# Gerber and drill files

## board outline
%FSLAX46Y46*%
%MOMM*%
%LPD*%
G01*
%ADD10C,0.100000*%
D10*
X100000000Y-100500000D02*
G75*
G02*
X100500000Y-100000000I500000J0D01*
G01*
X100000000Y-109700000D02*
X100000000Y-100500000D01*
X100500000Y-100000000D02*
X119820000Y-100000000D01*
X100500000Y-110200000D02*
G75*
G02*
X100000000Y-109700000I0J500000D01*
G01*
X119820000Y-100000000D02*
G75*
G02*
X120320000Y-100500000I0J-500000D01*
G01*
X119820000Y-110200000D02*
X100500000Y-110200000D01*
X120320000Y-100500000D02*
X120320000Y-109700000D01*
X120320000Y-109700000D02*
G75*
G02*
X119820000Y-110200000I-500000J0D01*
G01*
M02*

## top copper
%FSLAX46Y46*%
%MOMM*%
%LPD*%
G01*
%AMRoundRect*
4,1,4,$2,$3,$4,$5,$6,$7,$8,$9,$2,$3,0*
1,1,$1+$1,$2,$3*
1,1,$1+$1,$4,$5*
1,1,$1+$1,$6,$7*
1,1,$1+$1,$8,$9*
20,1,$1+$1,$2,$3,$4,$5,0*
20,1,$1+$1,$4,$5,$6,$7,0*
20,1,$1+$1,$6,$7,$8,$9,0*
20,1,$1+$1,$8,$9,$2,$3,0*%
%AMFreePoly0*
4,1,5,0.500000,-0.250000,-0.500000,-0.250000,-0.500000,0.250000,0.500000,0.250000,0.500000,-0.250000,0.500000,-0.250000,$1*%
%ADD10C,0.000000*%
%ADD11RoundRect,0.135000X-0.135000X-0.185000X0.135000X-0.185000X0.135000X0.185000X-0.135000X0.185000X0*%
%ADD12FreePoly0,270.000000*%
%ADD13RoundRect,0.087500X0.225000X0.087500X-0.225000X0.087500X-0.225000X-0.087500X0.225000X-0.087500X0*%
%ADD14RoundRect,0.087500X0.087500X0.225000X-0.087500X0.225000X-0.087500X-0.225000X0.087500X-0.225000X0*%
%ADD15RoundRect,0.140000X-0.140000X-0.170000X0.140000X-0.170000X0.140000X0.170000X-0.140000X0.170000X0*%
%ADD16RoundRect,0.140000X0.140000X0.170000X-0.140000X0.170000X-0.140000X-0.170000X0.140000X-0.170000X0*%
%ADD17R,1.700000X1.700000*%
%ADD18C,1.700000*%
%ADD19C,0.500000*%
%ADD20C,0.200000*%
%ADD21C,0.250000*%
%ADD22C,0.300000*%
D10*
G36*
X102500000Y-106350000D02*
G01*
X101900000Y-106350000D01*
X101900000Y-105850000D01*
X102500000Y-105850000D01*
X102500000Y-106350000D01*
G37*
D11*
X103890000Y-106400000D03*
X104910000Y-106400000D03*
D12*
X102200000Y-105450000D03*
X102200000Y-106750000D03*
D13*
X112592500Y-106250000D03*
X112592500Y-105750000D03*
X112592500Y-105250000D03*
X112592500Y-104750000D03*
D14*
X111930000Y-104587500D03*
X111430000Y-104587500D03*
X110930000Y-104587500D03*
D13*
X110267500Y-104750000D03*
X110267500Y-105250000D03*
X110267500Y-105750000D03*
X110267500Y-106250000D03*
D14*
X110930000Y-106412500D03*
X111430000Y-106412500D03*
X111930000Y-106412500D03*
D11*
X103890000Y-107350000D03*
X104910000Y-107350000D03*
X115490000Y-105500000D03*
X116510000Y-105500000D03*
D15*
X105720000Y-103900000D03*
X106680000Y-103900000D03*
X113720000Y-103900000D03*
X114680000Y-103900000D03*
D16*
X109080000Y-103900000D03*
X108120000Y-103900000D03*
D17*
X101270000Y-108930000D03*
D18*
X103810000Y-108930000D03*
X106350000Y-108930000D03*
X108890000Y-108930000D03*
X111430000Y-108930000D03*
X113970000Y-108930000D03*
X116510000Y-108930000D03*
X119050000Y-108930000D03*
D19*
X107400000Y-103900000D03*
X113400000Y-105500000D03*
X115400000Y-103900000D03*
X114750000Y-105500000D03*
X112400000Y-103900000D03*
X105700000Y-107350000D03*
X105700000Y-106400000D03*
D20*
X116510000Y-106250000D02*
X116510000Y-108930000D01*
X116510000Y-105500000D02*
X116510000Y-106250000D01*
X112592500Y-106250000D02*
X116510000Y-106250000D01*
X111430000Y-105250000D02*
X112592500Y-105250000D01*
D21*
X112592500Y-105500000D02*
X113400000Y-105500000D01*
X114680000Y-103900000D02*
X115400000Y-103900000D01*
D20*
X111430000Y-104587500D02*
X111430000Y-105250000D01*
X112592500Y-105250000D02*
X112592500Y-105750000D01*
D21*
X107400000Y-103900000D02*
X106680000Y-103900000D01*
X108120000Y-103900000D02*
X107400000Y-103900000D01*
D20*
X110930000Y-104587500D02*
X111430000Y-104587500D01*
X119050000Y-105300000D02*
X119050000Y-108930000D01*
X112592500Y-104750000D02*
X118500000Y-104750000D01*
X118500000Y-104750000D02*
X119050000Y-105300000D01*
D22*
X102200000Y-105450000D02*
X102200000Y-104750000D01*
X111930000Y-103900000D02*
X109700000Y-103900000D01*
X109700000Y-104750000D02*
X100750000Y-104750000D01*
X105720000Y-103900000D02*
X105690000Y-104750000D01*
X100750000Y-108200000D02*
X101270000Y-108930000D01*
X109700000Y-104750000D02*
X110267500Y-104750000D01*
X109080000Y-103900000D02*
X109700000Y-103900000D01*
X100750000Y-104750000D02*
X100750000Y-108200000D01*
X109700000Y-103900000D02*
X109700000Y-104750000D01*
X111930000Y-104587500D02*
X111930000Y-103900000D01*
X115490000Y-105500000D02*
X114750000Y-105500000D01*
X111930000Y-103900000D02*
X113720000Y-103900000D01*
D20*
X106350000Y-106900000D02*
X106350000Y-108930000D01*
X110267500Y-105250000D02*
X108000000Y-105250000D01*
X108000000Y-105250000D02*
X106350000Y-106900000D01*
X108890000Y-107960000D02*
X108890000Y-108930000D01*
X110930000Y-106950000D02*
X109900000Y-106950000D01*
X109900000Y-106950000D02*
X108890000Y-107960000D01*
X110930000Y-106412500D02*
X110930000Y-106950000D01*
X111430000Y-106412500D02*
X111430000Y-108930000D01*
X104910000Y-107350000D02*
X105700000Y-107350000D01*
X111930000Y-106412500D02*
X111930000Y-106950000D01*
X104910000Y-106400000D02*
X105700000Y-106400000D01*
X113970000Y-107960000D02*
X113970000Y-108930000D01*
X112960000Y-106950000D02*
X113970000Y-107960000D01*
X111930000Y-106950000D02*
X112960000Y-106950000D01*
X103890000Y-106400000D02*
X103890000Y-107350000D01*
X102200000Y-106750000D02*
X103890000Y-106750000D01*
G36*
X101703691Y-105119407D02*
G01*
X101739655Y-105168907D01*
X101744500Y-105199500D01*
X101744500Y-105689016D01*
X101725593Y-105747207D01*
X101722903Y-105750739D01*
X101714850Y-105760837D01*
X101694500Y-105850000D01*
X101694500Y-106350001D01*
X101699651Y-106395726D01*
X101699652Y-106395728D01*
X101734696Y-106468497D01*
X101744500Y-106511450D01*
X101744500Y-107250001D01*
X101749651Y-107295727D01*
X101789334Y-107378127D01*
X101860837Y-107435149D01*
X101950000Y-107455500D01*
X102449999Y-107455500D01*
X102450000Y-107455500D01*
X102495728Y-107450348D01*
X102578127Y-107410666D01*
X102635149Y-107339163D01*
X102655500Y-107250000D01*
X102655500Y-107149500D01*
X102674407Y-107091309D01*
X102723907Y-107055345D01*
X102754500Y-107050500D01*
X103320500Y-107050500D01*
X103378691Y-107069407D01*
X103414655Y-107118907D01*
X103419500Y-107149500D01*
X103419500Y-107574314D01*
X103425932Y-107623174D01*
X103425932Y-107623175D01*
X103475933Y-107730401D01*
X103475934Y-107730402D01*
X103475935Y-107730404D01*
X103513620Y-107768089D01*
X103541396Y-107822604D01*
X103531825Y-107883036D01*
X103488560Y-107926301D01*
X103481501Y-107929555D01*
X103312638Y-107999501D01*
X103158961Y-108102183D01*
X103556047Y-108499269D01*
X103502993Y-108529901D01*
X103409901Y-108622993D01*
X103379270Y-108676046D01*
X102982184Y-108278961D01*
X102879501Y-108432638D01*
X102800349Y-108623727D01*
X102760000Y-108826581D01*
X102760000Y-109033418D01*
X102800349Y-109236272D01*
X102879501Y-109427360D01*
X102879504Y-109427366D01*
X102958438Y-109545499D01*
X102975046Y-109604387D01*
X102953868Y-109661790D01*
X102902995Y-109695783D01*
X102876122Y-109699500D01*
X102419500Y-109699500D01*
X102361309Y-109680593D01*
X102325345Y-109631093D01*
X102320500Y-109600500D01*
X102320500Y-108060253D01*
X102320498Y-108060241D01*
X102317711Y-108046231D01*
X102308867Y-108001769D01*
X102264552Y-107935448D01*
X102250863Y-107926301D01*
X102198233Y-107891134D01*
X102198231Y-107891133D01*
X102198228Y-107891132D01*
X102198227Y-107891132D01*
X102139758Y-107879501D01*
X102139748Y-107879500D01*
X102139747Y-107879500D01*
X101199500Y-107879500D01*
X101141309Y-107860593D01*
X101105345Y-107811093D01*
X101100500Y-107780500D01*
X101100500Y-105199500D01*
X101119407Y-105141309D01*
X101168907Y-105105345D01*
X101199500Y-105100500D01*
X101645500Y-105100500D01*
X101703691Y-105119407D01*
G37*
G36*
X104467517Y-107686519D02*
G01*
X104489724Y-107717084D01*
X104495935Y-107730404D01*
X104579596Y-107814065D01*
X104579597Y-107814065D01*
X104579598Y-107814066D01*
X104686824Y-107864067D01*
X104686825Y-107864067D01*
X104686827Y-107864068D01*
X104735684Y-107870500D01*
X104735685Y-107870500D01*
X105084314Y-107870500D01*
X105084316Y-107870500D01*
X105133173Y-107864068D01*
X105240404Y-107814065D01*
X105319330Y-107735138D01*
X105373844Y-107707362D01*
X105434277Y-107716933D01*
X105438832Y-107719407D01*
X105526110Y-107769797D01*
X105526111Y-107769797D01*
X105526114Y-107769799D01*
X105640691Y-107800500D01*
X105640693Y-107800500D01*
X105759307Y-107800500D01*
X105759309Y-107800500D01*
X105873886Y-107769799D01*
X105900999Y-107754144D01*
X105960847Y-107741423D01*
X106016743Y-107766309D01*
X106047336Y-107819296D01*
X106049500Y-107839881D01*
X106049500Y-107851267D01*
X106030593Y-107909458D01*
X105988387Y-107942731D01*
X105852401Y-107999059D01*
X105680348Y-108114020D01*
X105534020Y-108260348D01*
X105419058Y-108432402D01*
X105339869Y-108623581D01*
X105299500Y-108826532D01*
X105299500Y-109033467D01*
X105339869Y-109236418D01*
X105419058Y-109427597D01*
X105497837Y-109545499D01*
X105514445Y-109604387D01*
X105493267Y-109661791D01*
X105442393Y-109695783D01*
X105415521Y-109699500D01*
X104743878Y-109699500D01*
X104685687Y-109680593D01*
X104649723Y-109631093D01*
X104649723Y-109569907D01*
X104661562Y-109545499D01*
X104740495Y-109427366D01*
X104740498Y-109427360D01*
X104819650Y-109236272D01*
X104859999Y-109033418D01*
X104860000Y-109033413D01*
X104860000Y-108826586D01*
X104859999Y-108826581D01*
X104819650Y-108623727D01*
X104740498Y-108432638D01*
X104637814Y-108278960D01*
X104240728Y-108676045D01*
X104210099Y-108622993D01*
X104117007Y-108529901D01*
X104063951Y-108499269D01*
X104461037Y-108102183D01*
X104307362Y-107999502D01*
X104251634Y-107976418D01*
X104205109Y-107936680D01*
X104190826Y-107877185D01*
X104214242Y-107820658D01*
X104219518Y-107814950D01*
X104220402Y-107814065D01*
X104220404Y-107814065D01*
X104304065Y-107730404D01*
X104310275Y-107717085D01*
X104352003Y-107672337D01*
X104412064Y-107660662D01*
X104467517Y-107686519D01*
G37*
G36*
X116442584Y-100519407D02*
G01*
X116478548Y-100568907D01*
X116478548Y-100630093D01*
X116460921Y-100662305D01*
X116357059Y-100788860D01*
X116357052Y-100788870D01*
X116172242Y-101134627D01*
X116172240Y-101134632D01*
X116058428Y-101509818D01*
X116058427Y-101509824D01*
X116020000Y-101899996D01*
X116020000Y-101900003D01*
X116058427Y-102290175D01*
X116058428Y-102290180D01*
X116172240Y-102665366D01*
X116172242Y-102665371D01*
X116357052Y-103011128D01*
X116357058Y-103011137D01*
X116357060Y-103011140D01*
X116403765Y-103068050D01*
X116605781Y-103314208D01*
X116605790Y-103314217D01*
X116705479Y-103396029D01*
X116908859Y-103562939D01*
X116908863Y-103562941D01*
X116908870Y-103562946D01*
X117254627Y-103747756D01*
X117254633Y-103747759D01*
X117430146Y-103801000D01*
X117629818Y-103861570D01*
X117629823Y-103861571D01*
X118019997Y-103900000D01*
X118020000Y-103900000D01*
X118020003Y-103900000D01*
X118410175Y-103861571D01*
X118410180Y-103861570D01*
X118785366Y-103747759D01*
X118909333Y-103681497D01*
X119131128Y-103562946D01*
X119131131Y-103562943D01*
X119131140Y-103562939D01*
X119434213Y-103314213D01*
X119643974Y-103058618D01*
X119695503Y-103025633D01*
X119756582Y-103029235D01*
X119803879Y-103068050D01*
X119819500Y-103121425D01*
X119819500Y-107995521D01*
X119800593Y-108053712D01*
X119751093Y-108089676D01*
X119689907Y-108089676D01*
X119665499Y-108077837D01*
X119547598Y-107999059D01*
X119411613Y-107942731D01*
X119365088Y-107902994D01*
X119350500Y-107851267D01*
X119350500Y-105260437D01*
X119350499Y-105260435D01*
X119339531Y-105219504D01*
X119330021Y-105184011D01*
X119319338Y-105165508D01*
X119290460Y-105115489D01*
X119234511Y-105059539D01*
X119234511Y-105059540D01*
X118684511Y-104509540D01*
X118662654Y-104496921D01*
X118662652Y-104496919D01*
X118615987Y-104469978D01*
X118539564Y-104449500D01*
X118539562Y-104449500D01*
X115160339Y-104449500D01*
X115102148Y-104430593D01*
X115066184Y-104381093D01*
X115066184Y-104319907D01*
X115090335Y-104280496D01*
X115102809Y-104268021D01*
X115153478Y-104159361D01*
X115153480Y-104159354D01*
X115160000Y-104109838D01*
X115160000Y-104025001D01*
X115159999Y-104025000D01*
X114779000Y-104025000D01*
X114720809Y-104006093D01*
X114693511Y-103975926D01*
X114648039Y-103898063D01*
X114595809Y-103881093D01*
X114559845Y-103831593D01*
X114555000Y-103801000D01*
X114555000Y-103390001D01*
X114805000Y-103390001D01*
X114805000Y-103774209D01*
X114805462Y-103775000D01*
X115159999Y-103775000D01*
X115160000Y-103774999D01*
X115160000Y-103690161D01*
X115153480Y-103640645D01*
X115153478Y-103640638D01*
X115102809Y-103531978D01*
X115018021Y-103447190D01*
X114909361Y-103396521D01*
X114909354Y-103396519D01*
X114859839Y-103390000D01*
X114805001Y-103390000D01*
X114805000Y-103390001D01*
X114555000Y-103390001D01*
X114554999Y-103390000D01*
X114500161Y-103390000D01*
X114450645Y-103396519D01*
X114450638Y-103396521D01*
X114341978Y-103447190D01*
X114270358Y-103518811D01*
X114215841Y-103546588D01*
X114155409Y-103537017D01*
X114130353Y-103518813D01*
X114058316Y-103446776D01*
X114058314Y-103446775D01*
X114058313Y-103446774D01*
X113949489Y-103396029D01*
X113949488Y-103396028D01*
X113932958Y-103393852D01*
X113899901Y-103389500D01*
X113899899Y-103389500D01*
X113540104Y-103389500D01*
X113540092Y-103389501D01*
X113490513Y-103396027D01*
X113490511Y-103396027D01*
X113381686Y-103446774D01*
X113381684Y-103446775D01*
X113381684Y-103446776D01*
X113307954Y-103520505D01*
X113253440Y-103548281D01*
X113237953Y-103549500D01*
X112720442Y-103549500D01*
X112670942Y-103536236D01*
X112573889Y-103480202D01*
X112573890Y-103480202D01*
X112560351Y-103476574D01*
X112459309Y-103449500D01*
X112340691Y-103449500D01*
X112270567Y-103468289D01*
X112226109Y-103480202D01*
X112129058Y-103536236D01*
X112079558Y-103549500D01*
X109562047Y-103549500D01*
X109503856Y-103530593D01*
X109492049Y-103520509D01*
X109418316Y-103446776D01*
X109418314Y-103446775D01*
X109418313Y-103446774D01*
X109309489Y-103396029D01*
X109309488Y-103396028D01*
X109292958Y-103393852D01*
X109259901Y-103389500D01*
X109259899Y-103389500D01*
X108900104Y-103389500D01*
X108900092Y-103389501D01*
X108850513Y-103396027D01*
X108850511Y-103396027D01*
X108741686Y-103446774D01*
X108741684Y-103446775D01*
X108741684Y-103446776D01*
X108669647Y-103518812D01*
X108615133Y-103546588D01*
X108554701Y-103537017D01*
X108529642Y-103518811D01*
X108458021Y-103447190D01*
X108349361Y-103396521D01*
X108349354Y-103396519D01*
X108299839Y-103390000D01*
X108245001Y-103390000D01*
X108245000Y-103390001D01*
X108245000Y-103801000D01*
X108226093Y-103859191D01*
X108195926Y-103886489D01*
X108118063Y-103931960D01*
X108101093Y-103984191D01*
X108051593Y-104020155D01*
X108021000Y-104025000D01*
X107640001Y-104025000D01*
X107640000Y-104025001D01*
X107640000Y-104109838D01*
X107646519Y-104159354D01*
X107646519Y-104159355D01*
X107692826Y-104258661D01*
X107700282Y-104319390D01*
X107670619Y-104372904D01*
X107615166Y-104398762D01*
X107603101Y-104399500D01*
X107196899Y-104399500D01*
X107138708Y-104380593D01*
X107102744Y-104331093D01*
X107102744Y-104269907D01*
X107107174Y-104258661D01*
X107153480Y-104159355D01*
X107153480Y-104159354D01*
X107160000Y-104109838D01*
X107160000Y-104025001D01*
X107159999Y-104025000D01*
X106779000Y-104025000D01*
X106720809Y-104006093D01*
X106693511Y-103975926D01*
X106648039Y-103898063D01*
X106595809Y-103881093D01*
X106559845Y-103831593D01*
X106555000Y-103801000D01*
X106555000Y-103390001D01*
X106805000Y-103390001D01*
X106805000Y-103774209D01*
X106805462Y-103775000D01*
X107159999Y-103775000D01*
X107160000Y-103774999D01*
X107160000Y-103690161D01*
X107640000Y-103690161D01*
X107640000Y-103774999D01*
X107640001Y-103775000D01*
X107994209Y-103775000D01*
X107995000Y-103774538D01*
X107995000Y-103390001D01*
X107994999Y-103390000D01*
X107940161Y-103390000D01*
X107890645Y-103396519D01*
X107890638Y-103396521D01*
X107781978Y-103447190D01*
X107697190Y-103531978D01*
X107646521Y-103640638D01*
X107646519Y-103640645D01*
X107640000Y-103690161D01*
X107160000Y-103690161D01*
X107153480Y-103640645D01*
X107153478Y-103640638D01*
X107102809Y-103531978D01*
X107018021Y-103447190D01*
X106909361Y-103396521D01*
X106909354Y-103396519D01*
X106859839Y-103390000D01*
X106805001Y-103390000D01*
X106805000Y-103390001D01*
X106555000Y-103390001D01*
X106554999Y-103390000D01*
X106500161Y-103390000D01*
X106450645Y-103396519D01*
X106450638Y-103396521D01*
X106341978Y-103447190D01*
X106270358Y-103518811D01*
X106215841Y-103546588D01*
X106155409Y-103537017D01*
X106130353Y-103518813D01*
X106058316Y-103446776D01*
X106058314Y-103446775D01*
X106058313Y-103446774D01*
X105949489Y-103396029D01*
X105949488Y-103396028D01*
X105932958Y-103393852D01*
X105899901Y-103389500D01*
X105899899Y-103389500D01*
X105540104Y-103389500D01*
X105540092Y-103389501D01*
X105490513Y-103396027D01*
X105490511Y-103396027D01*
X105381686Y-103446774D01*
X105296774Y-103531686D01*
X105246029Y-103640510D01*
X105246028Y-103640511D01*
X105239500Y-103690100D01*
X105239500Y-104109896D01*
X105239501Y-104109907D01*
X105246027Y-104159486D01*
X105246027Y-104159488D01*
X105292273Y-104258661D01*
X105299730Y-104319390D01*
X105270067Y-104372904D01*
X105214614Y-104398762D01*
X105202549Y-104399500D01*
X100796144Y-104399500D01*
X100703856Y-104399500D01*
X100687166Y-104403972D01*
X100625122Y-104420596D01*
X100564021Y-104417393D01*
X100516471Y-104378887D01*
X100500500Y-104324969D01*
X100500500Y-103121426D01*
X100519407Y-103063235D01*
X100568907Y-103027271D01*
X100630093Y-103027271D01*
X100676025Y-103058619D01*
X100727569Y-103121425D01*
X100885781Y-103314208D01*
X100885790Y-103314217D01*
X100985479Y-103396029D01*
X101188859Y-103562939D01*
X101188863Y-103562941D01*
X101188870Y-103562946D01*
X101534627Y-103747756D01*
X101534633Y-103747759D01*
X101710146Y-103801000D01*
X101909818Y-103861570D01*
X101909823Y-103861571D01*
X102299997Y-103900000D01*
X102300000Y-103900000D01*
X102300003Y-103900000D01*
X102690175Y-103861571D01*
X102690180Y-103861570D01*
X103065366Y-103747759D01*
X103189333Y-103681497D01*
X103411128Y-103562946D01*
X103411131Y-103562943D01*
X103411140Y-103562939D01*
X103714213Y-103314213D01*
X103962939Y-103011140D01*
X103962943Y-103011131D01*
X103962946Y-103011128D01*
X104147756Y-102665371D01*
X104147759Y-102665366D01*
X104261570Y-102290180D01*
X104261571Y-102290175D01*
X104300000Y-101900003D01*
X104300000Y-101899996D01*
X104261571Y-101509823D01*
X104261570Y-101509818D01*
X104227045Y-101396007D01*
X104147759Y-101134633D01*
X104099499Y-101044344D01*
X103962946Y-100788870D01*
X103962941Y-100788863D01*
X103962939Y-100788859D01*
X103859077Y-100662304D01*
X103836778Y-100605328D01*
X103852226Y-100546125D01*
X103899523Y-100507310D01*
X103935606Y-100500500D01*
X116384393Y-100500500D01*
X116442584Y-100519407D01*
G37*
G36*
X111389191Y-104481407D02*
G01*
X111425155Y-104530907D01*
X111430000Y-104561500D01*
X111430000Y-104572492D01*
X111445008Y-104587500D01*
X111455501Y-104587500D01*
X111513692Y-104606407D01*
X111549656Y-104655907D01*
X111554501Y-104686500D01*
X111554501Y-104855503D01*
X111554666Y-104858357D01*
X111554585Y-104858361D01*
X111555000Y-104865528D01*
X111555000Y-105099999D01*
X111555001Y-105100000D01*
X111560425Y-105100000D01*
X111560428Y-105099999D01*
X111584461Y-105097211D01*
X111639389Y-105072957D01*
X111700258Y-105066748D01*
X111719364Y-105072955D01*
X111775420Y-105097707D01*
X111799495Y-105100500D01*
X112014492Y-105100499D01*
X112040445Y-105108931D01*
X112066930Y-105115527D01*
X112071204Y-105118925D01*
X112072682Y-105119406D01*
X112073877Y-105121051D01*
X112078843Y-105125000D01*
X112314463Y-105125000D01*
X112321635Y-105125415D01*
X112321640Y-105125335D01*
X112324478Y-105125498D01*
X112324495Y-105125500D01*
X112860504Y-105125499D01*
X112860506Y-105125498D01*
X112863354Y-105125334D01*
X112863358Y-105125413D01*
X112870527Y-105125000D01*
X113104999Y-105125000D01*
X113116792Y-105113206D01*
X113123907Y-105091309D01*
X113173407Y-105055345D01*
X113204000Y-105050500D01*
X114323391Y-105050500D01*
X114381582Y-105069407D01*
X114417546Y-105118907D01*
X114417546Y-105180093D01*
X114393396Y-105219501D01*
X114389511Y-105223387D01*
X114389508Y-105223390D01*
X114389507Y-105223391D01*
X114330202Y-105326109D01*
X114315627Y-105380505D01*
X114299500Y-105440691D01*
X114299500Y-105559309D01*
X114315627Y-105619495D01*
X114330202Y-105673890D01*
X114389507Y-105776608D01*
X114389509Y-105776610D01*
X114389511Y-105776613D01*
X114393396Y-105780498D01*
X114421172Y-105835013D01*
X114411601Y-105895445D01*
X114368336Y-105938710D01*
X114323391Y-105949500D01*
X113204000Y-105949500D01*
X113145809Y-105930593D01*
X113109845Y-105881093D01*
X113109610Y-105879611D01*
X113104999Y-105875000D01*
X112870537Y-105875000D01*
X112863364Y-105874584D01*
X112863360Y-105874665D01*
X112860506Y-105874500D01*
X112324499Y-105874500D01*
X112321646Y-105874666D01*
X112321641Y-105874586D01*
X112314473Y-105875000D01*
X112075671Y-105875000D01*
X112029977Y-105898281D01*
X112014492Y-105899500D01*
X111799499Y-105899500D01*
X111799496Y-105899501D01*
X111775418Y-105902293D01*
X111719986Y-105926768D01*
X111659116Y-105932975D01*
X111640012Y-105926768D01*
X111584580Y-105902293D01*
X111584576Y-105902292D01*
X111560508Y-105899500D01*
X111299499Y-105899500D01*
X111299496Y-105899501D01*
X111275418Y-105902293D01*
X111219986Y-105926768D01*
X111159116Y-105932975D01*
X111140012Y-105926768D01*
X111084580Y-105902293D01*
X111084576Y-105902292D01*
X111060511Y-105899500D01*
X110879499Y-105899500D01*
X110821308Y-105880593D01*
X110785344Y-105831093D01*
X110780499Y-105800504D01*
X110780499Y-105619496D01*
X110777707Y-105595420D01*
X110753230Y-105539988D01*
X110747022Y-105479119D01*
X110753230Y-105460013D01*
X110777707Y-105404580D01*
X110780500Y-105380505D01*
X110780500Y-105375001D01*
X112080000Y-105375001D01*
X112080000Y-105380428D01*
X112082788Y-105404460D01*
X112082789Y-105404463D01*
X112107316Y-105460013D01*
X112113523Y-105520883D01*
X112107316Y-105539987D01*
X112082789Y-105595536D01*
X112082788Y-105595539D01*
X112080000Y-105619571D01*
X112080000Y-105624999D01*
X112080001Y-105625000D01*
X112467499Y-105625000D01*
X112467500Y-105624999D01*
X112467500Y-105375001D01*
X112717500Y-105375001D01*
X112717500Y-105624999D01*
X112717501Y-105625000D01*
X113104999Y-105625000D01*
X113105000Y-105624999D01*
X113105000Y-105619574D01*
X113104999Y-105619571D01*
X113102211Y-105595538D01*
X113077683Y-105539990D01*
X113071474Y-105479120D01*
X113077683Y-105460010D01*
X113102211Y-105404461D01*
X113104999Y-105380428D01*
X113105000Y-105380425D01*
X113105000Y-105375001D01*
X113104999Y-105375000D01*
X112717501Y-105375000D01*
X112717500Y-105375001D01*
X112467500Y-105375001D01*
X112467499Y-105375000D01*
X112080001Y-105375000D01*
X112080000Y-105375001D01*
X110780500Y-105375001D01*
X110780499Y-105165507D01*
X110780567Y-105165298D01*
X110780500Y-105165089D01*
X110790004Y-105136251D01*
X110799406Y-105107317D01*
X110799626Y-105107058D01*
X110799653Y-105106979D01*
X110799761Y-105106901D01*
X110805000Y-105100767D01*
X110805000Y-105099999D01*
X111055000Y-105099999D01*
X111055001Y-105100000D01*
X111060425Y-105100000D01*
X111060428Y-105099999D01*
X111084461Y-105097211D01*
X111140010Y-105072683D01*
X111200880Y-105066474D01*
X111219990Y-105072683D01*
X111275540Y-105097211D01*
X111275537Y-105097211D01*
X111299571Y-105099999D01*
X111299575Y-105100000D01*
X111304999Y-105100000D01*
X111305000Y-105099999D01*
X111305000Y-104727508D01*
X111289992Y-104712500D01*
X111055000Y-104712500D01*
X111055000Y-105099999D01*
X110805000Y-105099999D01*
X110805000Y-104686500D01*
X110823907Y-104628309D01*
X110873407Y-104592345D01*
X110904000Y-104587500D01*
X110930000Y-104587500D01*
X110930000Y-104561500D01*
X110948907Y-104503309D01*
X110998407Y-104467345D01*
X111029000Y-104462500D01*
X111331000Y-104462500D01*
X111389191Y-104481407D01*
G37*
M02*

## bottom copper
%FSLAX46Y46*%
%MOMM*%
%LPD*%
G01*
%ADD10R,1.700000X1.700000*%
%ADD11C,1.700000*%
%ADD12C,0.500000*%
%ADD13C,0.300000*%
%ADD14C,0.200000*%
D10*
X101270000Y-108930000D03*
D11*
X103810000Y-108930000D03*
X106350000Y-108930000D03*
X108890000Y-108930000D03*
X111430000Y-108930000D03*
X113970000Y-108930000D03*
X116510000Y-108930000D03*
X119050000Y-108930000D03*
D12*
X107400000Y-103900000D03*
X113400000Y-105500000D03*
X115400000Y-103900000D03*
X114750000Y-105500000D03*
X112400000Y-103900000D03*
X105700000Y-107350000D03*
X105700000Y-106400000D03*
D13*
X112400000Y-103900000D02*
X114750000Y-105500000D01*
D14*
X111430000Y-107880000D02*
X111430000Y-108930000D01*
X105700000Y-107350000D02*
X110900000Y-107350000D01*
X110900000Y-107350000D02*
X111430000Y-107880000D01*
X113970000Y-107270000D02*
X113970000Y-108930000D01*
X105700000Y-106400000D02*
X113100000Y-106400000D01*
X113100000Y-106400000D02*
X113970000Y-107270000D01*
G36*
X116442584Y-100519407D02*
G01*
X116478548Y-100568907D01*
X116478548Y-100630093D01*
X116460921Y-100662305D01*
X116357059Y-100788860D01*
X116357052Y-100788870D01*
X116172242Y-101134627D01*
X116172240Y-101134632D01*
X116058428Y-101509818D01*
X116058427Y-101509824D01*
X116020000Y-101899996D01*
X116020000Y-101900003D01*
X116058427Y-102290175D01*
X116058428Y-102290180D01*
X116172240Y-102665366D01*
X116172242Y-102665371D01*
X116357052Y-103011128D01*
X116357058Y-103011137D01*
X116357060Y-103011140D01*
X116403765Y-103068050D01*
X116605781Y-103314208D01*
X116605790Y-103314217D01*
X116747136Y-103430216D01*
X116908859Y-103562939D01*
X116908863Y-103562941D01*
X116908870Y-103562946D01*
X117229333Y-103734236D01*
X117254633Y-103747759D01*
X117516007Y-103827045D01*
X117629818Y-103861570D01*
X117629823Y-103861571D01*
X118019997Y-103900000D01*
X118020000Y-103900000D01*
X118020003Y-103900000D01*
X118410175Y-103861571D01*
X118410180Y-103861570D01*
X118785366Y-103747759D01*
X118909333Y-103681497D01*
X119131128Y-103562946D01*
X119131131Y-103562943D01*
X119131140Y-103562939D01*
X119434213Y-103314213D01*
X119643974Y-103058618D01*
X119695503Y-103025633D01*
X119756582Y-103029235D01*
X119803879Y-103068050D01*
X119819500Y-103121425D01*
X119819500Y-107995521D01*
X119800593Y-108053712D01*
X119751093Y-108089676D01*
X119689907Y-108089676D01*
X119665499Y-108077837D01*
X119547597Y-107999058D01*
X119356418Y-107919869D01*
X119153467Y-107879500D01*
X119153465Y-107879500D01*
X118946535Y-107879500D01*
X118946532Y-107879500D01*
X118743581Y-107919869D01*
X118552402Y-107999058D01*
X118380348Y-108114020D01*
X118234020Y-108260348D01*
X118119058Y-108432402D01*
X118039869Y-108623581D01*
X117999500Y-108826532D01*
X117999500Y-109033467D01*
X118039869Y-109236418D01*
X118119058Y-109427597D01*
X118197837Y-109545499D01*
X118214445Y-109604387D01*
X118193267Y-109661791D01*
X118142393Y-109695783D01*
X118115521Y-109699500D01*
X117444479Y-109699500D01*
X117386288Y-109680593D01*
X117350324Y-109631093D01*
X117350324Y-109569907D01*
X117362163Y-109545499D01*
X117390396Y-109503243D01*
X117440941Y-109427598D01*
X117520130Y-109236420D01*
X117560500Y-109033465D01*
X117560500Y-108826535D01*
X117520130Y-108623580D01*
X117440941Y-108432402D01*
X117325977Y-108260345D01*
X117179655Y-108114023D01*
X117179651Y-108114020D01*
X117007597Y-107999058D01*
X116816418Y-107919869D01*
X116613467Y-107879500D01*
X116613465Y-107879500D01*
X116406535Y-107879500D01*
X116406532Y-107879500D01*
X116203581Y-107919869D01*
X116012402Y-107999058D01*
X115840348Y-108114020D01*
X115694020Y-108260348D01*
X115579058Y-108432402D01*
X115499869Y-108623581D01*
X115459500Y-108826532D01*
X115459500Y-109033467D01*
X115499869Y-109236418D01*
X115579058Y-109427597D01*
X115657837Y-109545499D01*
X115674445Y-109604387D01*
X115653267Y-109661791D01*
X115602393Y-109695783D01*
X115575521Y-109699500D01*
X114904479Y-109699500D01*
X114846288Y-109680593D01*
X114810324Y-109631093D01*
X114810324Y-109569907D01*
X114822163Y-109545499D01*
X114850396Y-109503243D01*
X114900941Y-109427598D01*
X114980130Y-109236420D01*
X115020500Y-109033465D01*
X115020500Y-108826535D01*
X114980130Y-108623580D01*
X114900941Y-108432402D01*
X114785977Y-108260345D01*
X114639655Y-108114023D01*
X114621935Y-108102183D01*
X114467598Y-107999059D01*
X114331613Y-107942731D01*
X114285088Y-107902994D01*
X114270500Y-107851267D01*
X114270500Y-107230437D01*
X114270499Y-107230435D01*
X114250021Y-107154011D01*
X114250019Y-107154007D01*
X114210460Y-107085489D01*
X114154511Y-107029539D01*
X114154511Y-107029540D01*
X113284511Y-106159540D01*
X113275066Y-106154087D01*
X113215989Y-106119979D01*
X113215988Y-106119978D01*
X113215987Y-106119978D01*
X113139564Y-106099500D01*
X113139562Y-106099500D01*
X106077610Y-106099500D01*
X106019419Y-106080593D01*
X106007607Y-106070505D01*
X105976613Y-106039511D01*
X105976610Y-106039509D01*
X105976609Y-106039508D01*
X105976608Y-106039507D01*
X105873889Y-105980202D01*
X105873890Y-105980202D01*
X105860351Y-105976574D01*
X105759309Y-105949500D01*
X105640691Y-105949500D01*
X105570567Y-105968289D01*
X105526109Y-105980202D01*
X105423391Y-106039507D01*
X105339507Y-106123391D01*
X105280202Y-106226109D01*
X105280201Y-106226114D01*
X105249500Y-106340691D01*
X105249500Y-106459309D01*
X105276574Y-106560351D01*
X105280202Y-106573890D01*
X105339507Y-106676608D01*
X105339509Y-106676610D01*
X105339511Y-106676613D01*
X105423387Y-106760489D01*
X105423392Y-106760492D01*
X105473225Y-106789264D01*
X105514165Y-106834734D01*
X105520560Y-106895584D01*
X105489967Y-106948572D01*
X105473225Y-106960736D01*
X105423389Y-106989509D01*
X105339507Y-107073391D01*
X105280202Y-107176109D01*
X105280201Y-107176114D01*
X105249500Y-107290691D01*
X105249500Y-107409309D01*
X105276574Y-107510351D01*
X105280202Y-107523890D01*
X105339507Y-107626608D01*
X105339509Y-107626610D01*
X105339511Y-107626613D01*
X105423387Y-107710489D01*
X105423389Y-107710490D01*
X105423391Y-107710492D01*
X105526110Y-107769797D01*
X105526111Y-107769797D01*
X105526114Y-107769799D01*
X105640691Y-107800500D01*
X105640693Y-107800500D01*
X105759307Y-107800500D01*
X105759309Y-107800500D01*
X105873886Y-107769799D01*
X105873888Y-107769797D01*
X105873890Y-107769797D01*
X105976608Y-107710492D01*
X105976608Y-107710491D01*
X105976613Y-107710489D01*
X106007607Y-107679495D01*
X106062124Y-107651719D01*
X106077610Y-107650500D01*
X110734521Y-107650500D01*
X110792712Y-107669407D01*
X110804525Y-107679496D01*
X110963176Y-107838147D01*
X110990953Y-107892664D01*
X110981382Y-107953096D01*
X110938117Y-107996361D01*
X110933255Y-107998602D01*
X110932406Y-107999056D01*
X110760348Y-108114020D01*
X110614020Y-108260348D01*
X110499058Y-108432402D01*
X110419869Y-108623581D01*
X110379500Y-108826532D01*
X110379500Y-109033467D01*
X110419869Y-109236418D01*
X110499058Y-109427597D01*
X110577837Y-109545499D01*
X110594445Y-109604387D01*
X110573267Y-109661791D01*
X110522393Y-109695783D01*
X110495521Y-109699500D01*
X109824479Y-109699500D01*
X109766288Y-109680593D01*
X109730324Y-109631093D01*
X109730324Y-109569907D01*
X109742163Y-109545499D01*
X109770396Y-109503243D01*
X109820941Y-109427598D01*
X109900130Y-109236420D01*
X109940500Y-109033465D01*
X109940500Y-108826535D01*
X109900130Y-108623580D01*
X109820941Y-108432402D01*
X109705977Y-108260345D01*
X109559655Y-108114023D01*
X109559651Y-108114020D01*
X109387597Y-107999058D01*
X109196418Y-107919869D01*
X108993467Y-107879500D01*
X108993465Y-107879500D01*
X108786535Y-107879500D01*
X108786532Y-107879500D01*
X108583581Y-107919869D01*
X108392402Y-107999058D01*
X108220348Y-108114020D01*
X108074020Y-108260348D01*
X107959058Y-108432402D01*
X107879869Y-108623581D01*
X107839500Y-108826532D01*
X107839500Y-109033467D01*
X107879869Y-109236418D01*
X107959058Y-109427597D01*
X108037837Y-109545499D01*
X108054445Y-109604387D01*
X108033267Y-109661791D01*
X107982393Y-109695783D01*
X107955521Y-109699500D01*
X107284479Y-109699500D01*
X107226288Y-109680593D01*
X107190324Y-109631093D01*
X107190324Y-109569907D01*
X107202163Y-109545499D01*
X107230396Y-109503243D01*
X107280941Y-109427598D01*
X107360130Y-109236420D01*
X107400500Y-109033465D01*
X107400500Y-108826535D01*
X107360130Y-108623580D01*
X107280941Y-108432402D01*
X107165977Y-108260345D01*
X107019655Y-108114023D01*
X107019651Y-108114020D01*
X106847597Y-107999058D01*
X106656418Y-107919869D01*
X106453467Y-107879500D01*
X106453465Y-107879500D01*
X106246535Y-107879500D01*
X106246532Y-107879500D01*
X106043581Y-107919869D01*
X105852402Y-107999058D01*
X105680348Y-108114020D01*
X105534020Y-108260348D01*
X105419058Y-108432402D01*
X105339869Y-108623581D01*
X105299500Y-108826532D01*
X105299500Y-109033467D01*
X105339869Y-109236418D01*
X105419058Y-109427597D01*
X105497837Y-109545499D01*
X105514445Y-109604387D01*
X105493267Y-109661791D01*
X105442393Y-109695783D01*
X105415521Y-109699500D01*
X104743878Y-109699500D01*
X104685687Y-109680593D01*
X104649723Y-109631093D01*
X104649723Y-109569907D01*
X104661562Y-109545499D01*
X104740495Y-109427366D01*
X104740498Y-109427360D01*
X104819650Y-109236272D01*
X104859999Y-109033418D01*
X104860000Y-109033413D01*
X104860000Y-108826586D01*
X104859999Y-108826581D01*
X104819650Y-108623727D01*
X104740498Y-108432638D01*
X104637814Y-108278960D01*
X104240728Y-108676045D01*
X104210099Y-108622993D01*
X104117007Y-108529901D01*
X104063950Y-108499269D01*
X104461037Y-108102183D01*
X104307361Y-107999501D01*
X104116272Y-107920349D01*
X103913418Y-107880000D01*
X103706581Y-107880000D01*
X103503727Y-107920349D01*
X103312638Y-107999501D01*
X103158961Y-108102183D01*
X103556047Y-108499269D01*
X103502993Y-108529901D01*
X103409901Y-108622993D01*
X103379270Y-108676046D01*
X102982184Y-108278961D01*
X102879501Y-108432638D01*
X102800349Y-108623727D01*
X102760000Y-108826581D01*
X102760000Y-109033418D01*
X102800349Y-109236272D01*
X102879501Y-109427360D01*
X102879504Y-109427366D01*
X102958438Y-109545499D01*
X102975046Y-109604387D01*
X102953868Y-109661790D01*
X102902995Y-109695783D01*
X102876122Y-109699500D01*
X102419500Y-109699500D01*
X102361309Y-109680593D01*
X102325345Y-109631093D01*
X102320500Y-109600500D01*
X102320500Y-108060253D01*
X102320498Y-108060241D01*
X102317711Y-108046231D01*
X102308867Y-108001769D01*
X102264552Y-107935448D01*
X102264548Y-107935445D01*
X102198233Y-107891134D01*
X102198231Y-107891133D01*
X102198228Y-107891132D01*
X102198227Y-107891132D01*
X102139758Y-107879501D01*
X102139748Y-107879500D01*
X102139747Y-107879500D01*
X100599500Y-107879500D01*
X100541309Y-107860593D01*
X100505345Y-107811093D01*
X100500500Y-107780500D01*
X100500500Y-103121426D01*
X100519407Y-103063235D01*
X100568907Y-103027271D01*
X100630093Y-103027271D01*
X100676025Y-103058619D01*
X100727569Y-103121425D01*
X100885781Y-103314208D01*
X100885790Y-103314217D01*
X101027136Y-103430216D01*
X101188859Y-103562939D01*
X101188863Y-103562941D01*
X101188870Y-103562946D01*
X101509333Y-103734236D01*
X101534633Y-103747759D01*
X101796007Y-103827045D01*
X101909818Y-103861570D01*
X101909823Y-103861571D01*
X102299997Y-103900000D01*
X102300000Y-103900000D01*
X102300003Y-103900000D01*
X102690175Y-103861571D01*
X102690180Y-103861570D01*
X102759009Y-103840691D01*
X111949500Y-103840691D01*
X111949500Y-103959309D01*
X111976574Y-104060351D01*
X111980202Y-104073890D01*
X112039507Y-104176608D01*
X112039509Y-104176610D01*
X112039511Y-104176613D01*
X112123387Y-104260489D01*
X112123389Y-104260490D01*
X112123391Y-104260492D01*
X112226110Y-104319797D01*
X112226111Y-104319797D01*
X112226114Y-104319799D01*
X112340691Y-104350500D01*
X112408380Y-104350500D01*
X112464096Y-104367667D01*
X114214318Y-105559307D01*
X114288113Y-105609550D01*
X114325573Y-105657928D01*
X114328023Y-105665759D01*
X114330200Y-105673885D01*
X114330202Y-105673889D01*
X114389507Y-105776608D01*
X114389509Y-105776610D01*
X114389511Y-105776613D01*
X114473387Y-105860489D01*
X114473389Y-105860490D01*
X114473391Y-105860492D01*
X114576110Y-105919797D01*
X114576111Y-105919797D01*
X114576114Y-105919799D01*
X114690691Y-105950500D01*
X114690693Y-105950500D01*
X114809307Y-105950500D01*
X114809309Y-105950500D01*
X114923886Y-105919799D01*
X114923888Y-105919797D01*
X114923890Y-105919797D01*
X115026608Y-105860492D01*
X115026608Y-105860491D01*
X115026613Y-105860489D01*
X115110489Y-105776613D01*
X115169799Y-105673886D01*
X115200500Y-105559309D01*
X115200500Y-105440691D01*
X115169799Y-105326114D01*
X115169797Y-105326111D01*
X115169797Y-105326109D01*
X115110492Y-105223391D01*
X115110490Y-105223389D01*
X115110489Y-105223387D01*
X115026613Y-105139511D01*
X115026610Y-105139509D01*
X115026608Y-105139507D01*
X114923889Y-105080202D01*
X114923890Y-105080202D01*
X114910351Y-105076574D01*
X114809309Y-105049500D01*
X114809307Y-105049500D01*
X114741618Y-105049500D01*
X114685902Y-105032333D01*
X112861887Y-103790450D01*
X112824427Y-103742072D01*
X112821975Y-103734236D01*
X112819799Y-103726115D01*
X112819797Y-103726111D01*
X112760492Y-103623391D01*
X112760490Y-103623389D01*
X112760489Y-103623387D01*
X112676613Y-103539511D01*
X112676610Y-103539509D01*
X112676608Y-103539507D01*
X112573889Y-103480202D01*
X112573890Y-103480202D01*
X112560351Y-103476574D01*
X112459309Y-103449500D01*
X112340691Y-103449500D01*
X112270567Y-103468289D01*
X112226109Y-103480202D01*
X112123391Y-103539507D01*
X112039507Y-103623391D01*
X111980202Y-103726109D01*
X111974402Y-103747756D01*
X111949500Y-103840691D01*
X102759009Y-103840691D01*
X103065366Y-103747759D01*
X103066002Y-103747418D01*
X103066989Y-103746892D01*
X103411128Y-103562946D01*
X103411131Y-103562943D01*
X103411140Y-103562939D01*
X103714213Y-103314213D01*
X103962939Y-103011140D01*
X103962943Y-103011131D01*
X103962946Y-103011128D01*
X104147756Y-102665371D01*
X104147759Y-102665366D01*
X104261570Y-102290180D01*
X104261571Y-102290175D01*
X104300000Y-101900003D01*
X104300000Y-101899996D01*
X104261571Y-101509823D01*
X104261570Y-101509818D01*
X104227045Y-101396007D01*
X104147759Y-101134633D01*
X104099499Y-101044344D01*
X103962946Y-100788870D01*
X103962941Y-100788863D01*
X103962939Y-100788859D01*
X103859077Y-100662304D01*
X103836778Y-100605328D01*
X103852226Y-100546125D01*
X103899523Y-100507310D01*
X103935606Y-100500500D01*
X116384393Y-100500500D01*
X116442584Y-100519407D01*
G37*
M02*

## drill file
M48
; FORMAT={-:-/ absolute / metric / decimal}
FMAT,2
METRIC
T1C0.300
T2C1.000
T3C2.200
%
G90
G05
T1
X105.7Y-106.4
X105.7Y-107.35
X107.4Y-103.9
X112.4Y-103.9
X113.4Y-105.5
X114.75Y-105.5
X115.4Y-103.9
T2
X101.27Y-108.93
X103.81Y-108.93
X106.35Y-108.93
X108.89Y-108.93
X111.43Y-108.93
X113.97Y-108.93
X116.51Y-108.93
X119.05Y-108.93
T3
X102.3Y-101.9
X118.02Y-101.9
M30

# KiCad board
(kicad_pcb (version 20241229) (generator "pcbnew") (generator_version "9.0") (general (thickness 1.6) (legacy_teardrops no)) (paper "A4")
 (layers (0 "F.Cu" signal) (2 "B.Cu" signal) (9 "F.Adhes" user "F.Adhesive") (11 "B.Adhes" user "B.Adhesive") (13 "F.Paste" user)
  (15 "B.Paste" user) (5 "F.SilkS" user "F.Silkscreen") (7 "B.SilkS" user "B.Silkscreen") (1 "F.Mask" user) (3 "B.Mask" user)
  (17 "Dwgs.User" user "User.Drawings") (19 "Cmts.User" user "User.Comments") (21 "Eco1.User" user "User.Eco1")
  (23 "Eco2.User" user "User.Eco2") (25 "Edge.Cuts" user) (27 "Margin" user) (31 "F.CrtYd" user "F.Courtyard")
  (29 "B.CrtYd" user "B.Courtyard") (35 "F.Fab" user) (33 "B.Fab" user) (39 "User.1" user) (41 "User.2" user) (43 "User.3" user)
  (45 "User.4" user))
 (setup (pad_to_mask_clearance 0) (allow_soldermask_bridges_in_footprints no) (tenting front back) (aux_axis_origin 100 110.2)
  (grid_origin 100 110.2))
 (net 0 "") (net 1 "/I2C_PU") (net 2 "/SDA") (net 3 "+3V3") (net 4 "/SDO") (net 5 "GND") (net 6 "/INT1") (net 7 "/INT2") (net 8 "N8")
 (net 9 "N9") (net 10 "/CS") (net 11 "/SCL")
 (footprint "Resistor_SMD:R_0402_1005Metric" (layer "F.Cu") (at 104.4 106.4)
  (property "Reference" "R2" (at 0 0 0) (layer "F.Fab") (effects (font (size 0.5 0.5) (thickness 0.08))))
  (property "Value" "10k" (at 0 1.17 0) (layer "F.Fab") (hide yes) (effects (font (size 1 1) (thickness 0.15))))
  (pad "1" smd roundrect (at -0.51 0) (size 0.54 0.64) (layers "F.Cu" "F.Mask" "F.Paste") (roundrect_rratio 0.25) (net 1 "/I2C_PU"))
  (pad "2" smd roundrect (at 0.51 0) (size 0.54 0.64) (layers "F.Cu" "F.Mask" "F.Paste") (roundrect_rratio 0.25) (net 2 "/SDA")))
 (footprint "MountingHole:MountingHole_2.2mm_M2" (layer "F.Cu") (at 102.3 101.9)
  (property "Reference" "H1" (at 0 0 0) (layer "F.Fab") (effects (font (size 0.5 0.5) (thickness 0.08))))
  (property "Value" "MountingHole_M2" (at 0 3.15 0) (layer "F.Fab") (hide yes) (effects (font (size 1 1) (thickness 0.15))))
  (pad "" np_thru_hole circle (at 0 0) (size 2.2 2.2) (drill 2.2) (layers "*.Cu" "*.Mask")))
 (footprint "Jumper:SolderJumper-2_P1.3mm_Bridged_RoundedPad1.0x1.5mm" (layer "F.Cu") (at 102.2 106.1 -90)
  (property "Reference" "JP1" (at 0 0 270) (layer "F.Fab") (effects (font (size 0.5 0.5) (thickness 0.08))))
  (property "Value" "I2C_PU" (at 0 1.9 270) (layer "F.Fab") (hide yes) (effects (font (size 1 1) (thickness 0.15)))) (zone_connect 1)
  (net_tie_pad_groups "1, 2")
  (fp_poly (pts (xy 0.25 -0.3) (xy -0.25 -0.3) (xy -0.25 0.3) (xy 0.25 0.3)) (stroke (width 0) (type solid)) (fill yes) (layer "F.Cu"))
  (pad "1" smd custom (at -0.65 0 270) (size 1 0.5) (layers "F.Cu" "F.Mask") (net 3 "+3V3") (zone_connect 2) (thermal_bridge_angle 45)
   (options (clearance outline) (anchor rect)) (primitives))
  (pad "2" smd custom (at 0.65 0 270) (size 1 0.5) (layers "F.Cu" "F.Mask") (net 1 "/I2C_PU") (zone_connect 2) (thermal_bridge_angle 45)
   (options (clearance outline) (anchor rect)) (primitives)))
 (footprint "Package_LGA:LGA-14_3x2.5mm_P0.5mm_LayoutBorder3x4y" (layer "F.Cu") (at 111.43 105.5 180)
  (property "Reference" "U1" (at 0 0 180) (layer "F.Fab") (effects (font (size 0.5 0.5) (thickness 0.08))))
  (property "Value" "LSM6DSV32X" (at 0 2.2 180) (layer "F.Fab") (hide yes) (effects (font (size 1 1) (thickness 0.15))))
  (pad "1" smd roundrect (at -1.1625 -0.75 180) (size 0.625 0.35) (layers "F.Cu" "F.Mask" "F.Paste") (roundrect_rratio 0.25) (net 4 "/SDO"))
  (pad "2" smd roundrect (at -1.1625 -0.25 180) (size 0.625 0.35) (layers "F.Cu" "F.Mask" "F.Paste") (roundrect_rratio 0.25) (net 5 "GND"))
  (pad "3" smd roundrect (at -1.1625 0.25 180) (size 0.625 0.35) (layers "F.Cu" "F.Mask" "F.Paste") (roundrect_rratio 0.25) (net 5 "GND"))
  (pad "4" smd roundrect (at -1.1625 0.75 180) (size 0.625 0.35) (layers "F.Cu" "F.Mask" "F.Paste") (roundrect_rratio 0.25) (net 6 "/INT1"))
  (pad "5" smd roundrect (at -0.5 0.9125 180) (size 0.35 0.625) (layers "F.Cu" "F.Mask" "F.Paste") (roundrect_rratio 0.25) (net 3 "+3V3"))
  (pad "6" smd roundrect (at 0 0.9125 180) (size 0.35 0.625) (layers "F.Cu" "F.Mask" "F.Paste") (roundrect_rratio 0.25) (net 5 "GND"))
  (pad "7" smd roundrect (at 0.5 0.9125 180) (size 0.35 0.625) (layers "F.Cu" "F.Mask" "F.Paste") (roundrect_rratio 0.25) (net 5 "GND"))
  (pad "8" smd roundrect (at 1.1625 0.75 180) (size 0.625 0.35) (layers "F.Cu" "F.Mask" "F.Paste") (roundrect_rratio 0.25) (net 3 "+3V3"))
  (pad "9" smd roundrect (at 1.1625 0.25 180) (size 0.625 0.35) (layers "F.Cu" "F.Mask" "F.Paste") (roundrect_rratio 0.25) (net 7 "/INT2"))
  (pad "10" smd roundrect (at 1.1625 -0.25 180) (size 0.625 0.35) (layers "F.Cu" "F.Mask" "F.Paste") (roundrect_rratio 0.25) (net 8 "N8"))
  (pad "11" smd roundrect (at 1.1625 -0.75 180) (size 0.625 0.35) (layers "F.Cu" "F.Mask" "F.Paste") (roundrect_rratio 0.25) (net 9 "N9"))
  (pad "12" smd roundrect (at 0.5 -0.9125 180) (size 0.35 0.625) (layers "F.Cu" "F.Mask" "F.Paste") (roundrect_rratio 0.25) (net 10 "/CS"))
  (pad "13" smd roundrect (at 0 -0.9125 180) (size 0.35 0.625) (layers "F.Cu" "F.Mask" "F.Paste") (roundrect_rratio 0.25) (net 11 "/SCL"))
  (pad "14" smd roundrect (at -0.5 -0.9125 180) (size 0.35 0.625) (layers "F.Cu" "F.Mask" "F.Paste") (roundrect_rratio 0.25) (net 2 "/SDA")))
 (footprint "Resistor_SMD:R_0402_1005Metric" (layer "F.Cu") (at 104.4 107.35)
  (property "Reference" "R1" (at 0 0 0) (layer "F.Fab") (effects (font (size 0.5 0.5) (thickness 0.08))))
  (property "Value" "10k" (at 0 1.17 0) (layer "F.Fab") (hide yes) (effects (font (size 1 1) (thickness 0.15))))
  (pad "1" smd roundrect (at -0.51 0) (size 0.54 0.64) (layers "F.Cu" "F.Mask" "F.Paste") (roundrect_rratio 0.25) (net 1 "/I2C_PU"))
  (pad "2" smd roundrect (at 0.51 0) (size 0.54 0.64) (layers "F.Cu" "F.Mask" "F.Paste") (roundrect_rratio 0.25) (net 11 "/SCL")))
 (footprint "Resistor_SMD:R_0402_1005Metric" (layer "F.Cu") (at 116 105.5)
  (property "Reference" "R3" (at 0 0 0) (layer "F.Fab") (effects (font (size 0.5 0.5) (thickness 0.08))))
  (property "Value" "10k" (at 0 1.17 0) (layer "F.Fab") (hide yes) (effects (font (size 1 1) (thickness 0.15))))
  (pad "1" smd roundrect (at -0.51 0) (size 0.54 0.64) (layers "F.Cu" "F.Mask" "F.Paste") (roundrect_rratio 0.25) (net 3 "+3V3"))
  (pad "2" smd roundrect (at 0.51 0) (size 0.54 0.64) (layers "F.Cu" "F.Mask" "F.Paste") (roundrect_rratio 0.25) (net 4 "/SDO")))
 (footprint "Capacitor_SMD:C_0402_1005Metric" (layer "F.Cu") (at 106.2 103.9)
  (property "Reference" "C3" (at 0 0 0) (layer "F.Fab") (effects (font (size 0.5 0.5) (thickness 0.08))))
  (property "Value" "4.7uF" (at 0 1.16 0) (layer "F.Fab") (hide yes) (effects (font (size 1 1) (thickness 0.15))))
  (pad "1" smd roundrect (at -0.48 0) (size 0.56 0.62) (layers "F.Cu" "F.Mask" "F.Paste") (roundrect_rratio 0.25) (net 3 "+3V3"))
  (pad "2" smd roundrect (at 0.48 0) (size 0.56 0.62) (layers "F.Cu" "F.Mask" "F.Paste") (roundrect_rratio 0.25) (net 5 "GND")))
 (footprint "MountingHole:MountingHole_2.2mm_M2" (layer "F.Cu") (at 118.02 101.9)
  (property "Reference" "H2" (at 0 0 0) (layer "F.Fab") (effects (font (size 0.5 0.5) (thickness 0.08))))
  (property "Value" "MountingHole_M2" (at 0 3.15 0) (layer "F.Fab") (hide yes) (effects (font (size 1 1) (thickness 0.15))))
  (pad "" np_thru_hole circle (at 0 0) (size 2.2 2.2) (drill 2.2) (layers "*.Cu" "*.Mask")))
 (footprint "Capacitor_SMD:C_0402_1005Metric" (layer "F.Cu") (at 114.2 103.9)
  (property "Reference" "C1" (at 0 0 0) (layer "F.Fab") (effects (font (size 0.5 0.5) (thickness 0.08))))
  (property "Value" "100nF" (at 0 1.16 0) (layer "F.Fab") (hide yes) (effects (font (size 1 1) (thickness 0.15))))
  (pad "1" smd roundrect (at -0.48 0) (size 0.56 0.62) (layers "F.Cu" "F.Mask" "F.Paste") (roundrect_rratio 0.25) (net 3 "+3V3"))
  (pad "2" smd roundrect (at 0.48 0) (size 0.56 0.62) (layers "F.Cu" "F.Mask" "F.Paste") (roundrect_rratio 0.25) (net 5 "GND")))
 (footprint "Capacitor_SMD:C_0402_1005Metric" (layer "F.Cu") (at 108.6 103.9 180)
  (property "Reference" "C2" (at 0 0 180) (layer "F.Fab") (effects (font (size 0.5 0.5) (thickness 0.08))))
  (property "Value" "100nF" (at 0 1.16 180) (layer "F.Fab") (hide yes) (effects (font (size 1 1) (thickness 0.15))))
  (pad "1" smd roundrect (at -0.48 0 180) (size 0.56 0.62) (layers "F.Cu" "F.Mask" "F.Paste") (roundrect_rratio 0.25) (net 3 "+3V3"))
  (pad "2" smd roundrect (at 0.48 0 180) (size 0.56 0.62) (layers "F.Cu" "F.Mask" "F.Paste") (roundrect_rratio 0.25) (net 5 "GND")))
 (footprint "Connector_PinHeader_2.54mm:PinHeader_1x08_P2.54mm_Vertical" (layer "B.Cu") (at 101.27 108.93 -90)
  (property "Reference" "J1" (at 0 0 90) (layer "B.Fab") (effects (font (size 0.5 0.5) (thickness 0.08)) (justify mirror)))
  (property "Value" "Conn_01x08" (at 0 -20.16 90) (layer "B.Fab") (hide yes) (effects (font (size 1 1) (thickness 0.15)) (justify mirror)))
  (pad "1" thru_hole rect (at 0 0 270) (size 1.7 1.7) (drill 1) (layers "*.Cu" "*.Mask") (remove_unused_layers no) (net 3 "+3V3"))
  (pad "2" thru_hole circle (at 0 -2.54 270) (size 1.7 1.7) (drill 1) (layers "*.Cu" "*.Mask") (remove_unused_layers no) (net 5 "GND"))
  (pad "3" thru_hole circle (at 0 -5.08 270) (size 1.7 1.7) (drill 1) (layers "*.Cu" "*.Mask") (remove_unused_layers no) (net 7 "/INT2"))
  (pad "4" thru_hole circle (at 0 -7.62 270) (size 1.7 1.7) (drill 1) (layers "*.Cu" "*.Mask") (remove_unused_layers no) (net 10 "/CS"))
  (pad "5" thru_hole circle (at 0 -10.16 270) (size 1.7 1.7) (drill 1) (layers "*.Cu" "*.Mask") (remove_unused_layers no) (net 11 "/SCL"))
  (pad "6" thru_hole circle (at 0 -12.7 270) (size 1.7 1.7) (drill 1) (layers "*.Cu" "*.Mask") (remove_unused_layers no) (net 2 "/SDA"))
  (pad "7" thru_hole circle (at 0 -15.24 270) (size 1.7 1.7) (drill 1) (layers "*.Cu" "*.Mask") (remove_unused_layers no) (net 4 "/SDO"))
  (pad "8" thru_hole circle (at 0 -17.78 270) (size 1.7 1.7) (drill 1) (layers "*.Cu" "*.Mask") (remove_unused_layers no) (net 6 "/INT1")))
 (gr_arc (start 100 100.5) (mid 100.146446 100.146446) (end 100.5 100) (stroke (width 0.1) (type default)) (layer "Edge.Cuts"))
 (gr_line (start 100 109.7) (end 100 100.5) (stroke (width 0.1) (type default)) (layer "Edge.Cuts"))
 (gr_line (start 100.5 100) (end 119.82 100) (stroke (width 0.1) (type default)) (layer "Edge.Cuts"))
 (gr_arc (start 100.5 110.2) (mid 100.146446 110.053553) (end 100 109.7) (stroke (width 0.1) (type default)) (layer "Edge.Cuts"))
 (gr_arc (start 119.82 100) (mid 120.173553 100.146446) (end 120.32 100.5) (stroke (width 0.1) (type default)) (layer "Edge.Cuts"))
 (gr_line (start 119.82 110.2) (end 100.5 110.2) (stroke (width 0.1) (type default)) (layer "Edge.Cuts"))
 (gr_line (start 120.32 100.5) (end 120.32 109.7) (stroke (width 0.1) (type default)) (layer "Edge.Cuts"))
 (gr_arc (start 120.32 109.7) (mid 120.173553 110.053553) (end 119.82 110.2) (stroke (width 0.1) (type default)) (layer "Edge.Cuts"))
 (segment (start 116.51 106.25) (end 116.51 108.93) (width 0.2) (layer "F.Cu") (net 4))
 (segment (start 116.51 105.5) (end 116.51 106.25) (width 0.2) (layer "F.Cu") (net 4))
 (segment (start 112.5925 106.25) (end 116.51 106.25) (width 0.2) (layer "F.Cu") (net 4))
 (segment (start 111.43 105.25) (end 112.5925 105.25) (width 0.2) (layer "F.Cu") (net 5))
 (segment (start 112.5925 105.5) (end 113.4 105.5) (width 0.25) (layer "F.Cu") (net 5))
 (segment (start 114.68 103.9) (end 115.4 103.9) (width 0.25) (layer "F.Cu") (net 5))
 (segment (start 111.43 104.5875) (end 111.43 105.25) (width 0.2) (layer "F.Cu") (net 5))
 (segment (start 112.5925 105.25) (end 112.5925 105.75) (width 0.2) (layer "F.Cu") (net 5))
 (segment (start 107.4 103.9) (end 106.68 103.9) (width 0.25) (layer "F.Cu") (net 5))
 (segment (start 108.12 103.9) (end 107.4 103.9) (width 0.25) (layer "F.Cu") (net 5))
 (segment (start 110.93 104.5875) (end 111.43 104.5875) (width 0.2) (layer "F.Cu") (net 5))
 (via (at 107.4 103.9) (size 0.5) (drill 0.3) (layers "F.Cu" "B.Cu") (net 5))
 (via (at 113.4 105.5) (size 0.5) (drill 0.3) (layers "F.Cu" "B.Cu") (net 5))
 (via (at 115.4 103.9) (size 0.5) (drill 0.3) (layers "F.Cu" "B.Cu") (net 5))
 (segment (start 119.05 105.3) (end 119.05 108.93) (width 0.2) (layer "F.Cu") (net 6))
 (segment (start 112.5925 104.75) (end 118.5 104.75) (width 0.2) (layer "F.Cu") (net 6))
 (segment (start 118.5 104.75) (end 119.05 105.3) (width 0.2) (layer "F.Cu") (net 6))
 (segment (start 102.2 105.45) (end 102.2 104.75) (width 0.3) (layer "F.Cu") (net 3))
 (segment (start 111.93 103.9) (end 109.7 103.9) (width 0.3) (layer "F.Cu") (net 3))
 (segment (start 109.7 104.75) (end 100.75 104.75) (width 0.3) (layer "F.Cu") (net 3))
 (segment (start 105.72 103.9) (end 105.69 104.75) (width 0.3) (layer "F.Cu") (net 3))
 (segment (start 100.75 108.2) (end 101.27 108.93) (width 0.3) (layer "F.Cu") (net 3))
 (segment (start 109.7 104.75) (end 110.2675 104.75) (width 0.3) (layer "F.Cu") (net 3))
 (segment (start 109.08 103.9) (end 109.7 103.9) (width 0.3) (layer "F.Cu") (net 3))
 (segment (start 100.75 104.75) (end 100.75 108.2) (width 0.3) (layer "F.Cu") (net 3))
 (segment (start 109.7 103.9) (end 109.7 104.75) (width 0.3) (layer "F.Cu") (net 3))
 (segment (start 111.93 104.5875) (end 111.93 103.9) (width 0.3) (layer "F.Cu") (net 3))
 (segment (start 115.49 105.5) (end 114.75 105.5) (width 0.3) (layer "F.Cu") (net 3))
 (segment (start 111.93 103.9) (end 113.72 103.9) (width 0.3) (layer "F.Cu") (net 3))
 (via (at 114.75 105.5) (size 0.5) (drill 0.3) (layers "F.Cu" "B.Cu") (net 3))
 (via (at 112.4 103.9) (size 0.5) (drill 0.3) (layers "F.Cu" "B.Cu") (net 3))
 (segment (start 112.4 103.9) (end 114.75 105.5) (width 0.3) (layer "B.Cu") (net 3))
 (segment (start 106.35 106.9) (end 106.35 108.93) (width 0.2) (layer "F.Cu") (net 7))
 (segment (start 110.2675 105.25) (end 108 105.25) (width 0.2) (layer "F.Cu") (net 7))
 (segment (start 108 105.25) (end 106.35 106.9) (width 0.2) (layer "F.Cu") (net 7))
 (segment (start 108.89 107.96) (end 108.89 108.93) (width 0.2) (layer "F.Cu") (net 10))
 (segment (start 110.93 106.95) (end 109.9 106.95) (width 0.2) (layer "F.Cu") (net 10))
 (segment (start 109.9 106.95) (end 108.89 107.96) (width 0.2) (layer "F.Cu") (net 10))
 (segment (start 110.93 106.4125) (end 110.93 106.95) (width 0.2) (layer "F.Cu") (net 10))
 (segment (start 111.43 106.4125) (end 111.43 108.93) (width 0.2) (layer "F.Cu") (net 11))
 (segment (start 104.91 107.35) (end 105.7 107.35) (width 0.2) (layer "F.Cu") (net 11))
 (via (at 105.7 107.35) (size 0.5) (drill 0.3) (layers "F.Cu" "B.Cu") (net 11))
 (segment (start 111.43 107.88) (end 111.43 108.93) (width 0.2) (layer "B.Cu") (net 11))
 (segment (start 105.7 107.35) (end 110.9 107.35) (width 0.2) (layer "B.Cu") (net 11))
 (segment (start 110.9 107.35) (end 111.43 107.88) (width 0.2) (layer "B.Cu") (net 11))
 (segment (start 111.93 106.4125) (end 111.93 106.95) (width 0.2) (layer "F.Cu") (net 2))
 (segment (start 104.91 106.4) (end 105.7 106.4) (width 0.2) (layer "F.Cu") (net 2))
 (segment (start 113.97 107.96) (end 113.97 108.93) (width 0.2) (layer "F.Cu") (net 2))
 (segment (start 112.96 106.95) (end 113.97 107.96) (width 0.2) (layer "F.Cu") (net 2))
 (segment (start 111.93 106.95) (end 112.96 106.95) (width 0.2) (layer "F.Cu") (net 2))
 (via (at 105.7 106.4) (size 0.5) (drill 0.3) (layers "F.Cu" "B.Cu") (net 2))
 (segment (start 113.97 107.27) (end 113.97 108.93) (width 0.2) (layer "B.Cu") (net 2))
 (segment (start 105.7 106.4) (end 113.1 106.4) (width 0.2) (layer "B.Cu") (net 2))
 (segment (start 113.1 106.4) (end 113.97 107.27) (width 0.2) (layer "B.Cu") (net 2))
 (segment (start 103.89 106.4) (end 103.89 107.35) (width 0.2) (layer "F.Cu") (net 1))
 (segment (start 102.2 106.75) (end 103.89 106.75) (width 0.2) (layer "F.Cu") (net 1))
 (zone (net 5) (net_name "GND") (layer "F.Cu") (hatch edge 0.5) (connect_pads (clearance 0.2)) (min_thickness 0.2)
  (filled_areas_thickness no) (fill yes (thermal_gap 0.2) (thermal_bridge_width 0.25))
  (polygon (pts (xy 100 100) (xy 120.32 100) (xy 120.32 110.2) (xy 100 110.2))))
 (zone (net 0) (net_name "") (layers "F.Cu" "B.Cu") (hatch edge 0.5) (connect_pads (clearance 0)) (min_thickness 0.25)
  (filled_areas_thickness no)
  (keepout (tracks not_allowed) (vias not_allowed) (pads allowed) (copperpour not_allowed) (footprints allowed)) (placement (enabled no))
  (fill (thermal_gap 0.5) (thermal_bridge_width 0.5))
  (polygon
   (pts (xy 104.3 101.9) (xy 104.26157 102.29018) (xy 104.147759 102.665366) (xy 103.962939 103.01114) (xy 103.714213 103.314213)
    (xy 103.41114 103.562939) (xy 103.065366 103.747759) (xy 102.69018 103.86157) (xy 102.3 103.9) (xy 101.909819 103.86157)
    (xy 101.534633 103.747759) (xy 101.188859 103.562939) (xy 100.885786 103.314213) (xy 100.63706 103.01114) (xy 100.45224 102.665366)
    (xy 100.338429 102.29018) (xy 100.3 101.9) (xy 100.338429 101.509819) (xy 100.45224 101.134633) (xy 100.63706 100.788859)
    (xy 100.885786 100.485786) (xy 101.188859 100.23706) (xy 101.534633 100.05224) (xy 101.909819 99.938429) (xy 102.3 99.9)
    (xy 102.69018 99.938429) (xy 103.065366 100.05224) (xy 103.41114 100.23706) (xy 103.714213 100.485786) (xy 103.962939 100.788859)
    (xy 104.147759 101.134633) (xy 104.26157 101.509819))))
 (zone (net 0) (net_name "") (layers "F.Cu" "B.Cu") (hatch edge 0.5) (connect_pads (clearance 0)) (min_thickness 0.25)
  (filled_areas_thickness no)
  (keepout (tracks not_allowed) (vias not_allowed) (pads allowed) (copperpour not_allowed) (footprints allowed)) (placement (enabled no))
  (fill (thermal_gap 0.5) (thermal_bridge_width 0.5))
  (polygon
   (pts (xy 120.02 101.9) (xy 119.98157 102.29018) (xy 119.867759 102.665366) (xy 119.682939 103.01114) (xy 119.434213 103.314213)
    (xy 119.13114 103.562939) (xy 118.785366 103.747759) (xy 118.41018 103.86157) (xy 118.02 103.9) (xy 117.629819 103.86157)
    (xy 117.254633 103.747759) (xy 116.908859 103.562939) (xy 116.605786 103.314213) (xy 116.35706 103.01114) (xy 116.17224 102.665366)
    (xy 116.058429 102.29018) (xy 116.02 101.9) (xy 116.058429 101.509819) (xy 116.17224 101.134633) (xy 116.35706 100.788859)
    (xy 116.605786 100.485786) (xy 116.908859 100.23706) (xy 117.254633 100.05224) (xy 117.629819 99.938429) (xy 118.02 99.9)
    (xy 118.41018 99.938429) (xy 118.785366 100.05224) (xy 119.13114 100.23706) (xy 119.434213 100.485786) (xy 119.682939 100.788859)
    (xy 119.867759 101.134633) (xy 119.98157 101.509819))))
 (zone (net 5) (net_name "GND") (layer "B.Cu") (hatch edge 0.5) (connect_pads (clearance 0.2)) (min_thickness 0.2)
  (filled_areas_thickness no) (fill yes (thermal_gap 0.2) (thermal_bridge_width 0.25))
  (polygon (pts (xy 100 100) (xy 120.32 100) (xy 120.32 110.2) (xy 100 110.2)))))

